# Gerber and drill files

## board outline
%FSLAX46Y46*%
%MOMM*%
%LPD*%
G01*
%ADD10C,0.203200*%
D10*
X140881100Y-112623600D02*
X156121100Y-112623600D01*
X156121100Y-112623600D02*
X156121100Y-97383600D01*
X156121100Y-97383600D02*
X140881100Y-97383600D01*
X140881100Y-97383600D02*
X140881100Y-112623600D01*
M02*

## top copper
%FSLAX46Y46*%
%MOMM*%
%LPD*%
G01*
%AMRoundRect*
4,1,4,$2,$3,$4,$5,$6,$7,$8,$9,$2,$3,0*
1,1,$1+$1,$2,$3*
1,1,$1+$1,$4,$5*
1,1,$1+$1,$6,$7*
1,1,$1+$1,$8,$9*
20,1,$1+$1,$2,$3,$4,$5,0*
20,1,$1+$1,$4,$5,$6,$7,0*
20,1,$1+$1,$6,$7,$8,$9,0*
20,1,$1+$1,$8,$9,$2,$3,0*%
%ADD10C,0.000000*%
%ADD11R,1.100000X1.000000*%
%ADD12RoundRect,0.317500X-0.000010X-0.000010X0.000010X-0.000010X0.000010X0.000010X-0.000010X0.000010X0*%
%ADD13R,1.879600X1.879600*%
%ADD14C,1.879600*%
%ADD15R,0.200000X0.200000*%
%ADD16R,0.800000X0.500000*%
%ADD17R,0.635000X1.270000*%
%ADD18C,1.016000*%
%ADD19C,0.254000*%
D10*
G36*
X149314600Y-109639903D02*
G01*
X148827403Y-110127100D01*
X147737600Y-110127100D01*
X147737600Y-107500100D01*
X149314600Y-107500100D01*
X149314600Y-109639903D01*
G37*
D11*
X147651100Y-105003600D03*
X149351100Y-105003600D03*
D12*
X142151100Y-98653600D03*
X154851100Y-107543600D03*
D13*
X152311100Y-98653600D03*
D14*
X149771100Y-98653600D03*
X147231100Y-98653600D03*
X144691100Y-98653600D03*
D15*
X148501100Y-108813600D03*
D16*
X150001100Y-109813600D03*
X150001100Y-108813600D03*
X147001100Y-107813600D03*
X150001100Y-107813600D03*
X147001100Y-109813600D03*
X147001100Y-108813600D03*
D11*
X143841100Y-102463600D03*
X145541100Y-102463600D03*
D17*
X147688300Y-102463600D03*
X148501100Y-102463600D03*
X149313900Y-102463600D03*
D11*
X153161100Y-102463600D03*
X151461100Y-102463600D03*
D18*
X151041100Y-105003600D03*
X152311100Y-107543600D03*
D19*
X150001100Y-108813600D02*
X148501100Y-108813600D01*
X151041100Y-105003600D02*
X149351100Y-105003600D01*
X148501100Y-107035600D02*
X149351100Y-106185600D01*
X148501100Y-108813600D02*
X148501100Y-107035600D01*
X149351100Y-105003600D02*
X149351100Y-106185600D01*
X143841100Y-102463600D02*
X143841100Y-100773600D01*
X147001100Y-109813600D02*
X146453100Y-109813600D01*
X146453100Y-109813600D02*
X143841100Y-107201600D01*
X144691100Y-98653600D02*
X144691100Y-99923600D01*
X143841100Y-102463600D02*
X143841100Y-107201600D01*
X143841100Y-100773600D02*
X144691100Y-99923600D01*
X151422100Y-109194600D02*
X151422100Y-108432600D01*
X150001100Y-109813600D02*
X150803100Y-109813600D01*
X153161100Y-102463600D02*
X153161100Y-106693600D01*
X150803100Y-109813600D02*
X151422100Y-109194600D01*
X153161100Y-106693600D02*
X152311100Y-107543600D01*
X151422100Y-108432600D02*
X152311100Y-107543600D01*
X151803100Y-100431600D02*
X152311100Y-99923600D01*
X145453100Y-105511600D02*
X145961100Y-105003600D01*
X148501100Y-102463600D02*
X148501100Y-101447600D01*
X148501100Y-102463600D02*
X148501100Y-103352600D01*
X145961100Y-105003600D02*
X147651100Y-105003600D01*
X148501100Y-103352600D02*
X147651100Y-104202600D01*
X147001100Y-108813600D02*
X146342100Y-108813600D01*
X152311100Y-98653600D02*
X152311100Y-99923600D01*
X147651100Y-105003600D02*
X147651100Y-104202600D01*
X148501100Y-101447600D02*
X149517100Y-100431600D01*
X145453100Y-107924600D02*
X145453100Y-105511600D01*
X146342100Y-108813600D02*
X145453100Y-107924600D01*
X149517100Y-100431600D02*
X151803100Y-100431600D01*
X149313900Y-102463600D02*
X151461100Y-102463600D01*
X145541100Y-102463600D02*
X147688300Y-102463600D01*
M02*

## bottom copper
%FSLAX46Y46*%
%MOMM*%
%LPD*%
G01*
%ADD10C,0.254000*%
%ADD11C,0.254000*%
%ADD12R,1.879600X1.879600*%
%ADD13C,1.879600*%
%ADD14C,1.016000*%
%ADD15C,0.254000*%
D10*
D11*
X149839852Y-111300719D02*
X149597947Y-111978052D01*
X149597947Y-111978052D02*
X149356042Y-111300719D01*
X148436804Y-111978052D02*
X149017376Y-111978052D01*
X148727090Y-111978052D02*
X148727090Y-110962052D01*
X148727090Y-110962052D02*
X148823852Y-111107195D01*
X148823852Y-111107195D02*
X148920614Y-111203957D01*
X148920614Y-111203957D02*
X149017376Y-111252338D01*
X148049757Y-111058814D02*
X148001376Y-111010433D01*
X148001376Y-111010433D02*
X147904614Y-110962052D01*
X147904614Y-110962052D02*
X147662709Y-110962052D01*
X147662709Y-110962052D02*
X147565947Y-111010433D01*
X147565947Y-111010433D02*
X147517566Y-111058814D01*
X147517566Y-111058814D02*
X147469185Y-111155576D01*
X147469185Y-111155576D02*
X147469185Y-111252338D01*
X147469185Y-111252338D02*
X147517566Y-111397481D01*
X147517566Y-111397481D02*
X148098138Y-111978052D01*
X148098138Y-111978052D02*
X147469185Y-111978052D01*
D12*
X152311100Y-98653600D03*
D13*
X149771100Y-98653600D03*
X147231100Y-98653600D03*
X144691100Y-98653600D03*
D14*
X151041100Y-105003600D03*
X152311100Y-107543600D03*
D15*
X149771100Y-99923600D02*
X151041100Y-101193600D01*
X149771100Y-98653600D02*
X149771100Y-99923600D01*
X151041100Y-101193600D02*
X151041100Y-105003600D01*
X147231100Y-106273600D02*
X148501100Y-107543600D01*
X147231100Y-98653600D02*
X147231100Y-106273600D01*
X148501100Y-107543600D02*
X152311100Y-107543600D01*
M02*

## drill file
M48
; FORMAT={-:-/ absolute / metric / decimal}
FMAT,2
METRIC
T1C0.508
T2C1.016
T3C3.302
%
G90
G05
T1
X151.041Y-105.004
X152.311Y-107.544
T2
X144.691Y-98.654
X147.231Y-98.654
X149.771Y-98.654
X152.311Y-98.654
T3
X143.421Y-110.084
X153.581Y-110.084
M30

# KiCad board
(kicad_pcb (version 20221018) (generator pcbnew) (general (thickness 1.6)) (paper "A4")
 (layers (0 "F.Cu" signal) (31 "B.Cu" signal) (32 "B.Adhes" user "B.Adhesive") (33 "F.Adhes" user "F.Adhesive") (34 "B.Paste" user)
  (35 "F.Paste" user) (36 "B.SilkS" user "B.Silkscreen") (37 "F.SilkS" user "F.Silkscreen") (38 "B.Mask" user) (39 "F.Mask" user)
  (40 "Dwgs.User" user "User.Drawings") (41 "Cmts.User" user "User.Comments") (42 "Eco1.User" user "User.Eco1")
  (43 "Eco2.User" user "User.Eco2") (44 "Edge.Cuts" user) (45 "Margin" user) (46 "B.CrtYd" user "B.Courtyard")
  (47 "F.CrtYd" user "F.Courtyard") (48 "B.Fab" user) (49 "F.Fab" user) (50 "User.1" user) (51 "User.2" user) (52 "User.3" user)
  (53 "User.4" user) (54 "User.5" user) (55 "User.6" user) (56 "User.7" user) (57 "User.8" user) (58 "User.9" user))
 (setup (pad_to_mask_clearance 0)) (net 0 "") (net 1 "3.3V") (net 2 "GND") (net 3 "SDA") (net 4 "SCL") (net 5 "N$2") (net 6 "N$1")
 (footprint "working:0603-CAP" (layer "F.Cu") (at 148.5011 105.0036)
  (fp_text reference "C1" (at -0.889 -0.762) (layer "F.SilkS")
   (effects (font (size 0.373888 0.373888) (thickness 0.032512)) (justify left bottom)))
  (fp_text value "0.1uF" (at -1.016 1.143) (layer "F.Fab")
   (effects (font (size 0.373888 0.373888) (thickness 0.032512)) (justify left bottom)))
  (pad "1" smd rect (at -0.85 0) (size 1.1 1) (layers "F.Cu" "F.Paste" "F.Mask") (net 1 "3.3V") (solder_mask_margin 0.1016)
   (thermal_bridge_angle 45))
  (pad "2" smd rect (at 0.85 0) (size 1.1 1) (layers "F.Cu" "F.Paste" "F.Mask") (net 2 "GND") (solder_mask_margin 0.1016)
   (thermal_bridge_angle 45)))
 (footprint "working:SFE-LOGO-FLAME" (layer "F.Cu") (at 153.42235 106.2101)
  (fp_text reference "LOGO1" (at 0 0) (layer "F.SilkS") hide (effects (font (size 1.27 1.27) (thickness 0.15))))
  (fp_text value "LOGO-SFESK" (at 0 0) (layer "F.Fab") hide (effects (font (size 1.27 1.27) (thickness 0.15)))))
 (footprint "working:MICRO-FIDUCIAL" (layer "F.Cu") (at 142.1511 98.6536)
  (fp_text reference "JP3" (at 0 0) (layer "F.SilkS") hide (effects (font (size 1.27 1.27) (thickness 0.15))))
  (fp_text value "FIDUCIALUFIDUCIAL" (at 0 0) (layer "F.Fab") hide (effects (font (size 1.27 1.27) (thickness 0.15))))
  (pad "1" smd roundrect (at 0 0) (size 0.635 0.635) (layers "F.Cu" "F.Mask") (roundrect_rratio 0.5) (solder_mask_margin 0.1016)
   (thermal_bridge_angle 45)))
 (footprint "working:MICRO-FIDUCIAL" (layer "F.Cu") (at 154.8511 107.5436)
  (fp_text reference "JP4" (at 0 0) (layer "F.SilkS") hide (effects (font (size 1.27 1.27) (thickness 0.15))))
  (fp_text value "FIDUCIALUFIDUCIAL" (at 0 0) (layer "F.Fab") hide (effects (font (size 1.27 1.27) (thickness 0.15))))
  (pad "1" smd roundrect (at 0 0) (size 0.635 0.635) (layers "F.Cu" "F.Mask") (roundrect_rratio 0.5) (solder_mask_margin 0.1016)
   (thermal_bridge_angle 45)))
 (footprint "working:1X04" (layer "F.Cu") (at 152.3111 98.6536 180)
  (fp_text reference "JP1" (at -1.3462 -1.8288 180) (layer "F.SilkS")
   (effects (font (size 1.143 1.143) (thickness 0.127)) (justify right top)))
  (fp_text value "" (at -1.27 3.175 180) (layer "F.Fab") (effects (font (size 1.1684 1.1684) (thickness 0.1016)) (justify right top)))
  (pad "1" thru_hole rect (at 0 0 270) (size 1.8796 1.8796) (drill 1.016) (layers "*.Cu" "*.Mask") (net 1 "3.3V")
   (solder_mask_margin 0.1016) (thermal_bridge_angle 45))
  (pad "2" thru_hole circle (at 2.54 0 270) (size 1.8796 1.8796) (drill 1.016) (layers "*.Cu" "*.Mask") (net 2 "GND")
   (solder_mask_margin 0.1016))
  (pad "3" thru_hole circle (at 5.08 0 270) (size 1.8796 1.8796) (drill 1.016) (layers "*.Cu" "*.Mask") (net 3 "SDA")
   (solder_mask_margin 0.1016))
  (pad "4" thru_hole circle (at 7.62 0 270) (size 1.8796 1.8796) (drill 1.016) (layers "*.Cu" "*.Mask") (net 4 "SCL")
   (solder_mask_margin 0.1016)))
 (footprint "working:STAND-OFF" (layer "F.Cu") (at 153.5811 110.0836)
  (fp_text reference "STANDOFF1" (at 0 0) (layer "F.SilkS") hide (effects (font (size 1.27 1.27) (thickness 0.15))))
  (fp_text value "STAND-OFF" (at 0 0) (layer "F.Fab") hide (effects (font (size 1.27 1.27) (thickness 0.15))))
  (pad "" np_thru_hole circle (at 0 0) (size 3.302 3.302) (drill 3.302) (layers "*.Cu" "*.Mask")))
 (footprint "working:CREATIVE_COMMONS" (layer "F.Cu") (at 128.1811 121.5136)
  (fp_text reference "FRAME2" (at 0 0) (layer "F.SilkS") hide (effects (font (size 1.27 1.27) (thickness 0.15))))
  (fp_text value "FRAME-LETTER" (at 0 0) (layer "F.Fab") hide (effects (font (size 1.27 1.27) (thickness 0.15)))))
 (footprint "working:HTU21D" (layer "F.Cu") (at 148.5011 108.8136)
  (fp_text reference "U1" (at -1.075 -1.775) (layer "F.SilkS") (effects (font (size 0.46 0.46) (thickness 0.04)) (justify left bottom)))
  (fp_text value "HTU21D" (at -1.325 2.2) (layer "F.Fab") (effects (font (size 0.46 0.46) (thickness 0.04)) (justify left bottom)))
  (fp_poly
   (pts (xy 0.8135 0.826303) (xy 0.326303 1.3135) (xy -0.7635 1.3135) (xy -0.7635 -1.3135) (xy 0.8135 -1.3135))
   (stroke (width 0) (type default)) (fill solid) (layer "F.Cu"))
  (pad "7" smd rect (at 0 0) (size 0.2 0.2) (layers "F.Cu" "F.Paste" "F.Mask") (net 2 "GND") (solder_mask_margin 0.1016)
   (thermal_bridge_angle 45))
  (pad "DATA" smd rect (at 1.5 1 270) (size 0.5 0.8) (layers "F.Cu" "F.Paste" "F.Mask") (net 3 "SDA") (solder_mask_margin 0.1016)
   (thermal_bridge_angle 45))
  (pad "GND" smd rect (at 1.5 0 270) (size 0.5 0.8) (layers "F.Cu" "F.Paste" "F.Mask") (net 2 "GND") (solder_mask_margin 0.1016)
   (thermal_bridge_angle 45))
  (pad "NC@1" smd rect (at -1.5 -1 270) (size 0.5 0.8) (layers "F.Cu" "F.Paste" "F.Mask") (solder_mask_margin 0.1016)
   (thermal_bridge_angle 45))
  (pad "NC@6" smd rect (at 1.5 -1 270) (size 0.5 0.8) (layers "F.Cu" "F.Paste" "F.Mask") (solder_mask_margin 0.1016)
   (thermal_bridge_angle 45))
  (pad "SCK" smd rect (at -1.5 1 270) (size 0.5 0.8) (layers "F.Cu" "F.Paste" "F.Mask") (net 4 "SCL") (solder_mask_margin 0.1016)
   (thermal_bridge_angle 45))
  (pad "VDD" smd rect (at -1.5 0 270) (size 0.5 0.8) (layers "F.Cu" "F.Paste" "F.Mask") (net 1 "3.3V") (solder_mask_margin 0.1016)
   (thermal_bridge_angle 45)))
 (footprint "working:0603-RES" (layer "F.Cu") (at 144.6911 102.4636)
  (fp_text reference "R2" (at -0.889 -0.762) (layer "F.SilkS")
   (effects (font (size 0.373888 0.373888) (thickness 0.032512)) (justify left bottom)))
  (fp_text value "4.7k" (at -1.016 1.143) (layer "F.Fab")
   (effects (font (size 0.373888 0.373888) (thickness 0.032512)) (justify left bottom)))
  (pad "1" smd rect (at -0.85 0) (size 1.1 1) (layers "F.Cu" "F.Paste" "F.Mask") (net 4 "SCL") (solder_mask_margin 0.1016)
   (thermal_bridge_angle 45))
  (pad "2" smd rect (at 0.85 0) (size 1.1 1) (layers "F.Cu" "F.Paste" "F.Mask") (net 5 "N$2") (solder_mask_margin 0.1016)
   (thermal_bridge_angle 45)))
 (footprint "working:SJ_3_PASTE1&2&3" (layer "F.Cu") (at 148.5011 102.4636)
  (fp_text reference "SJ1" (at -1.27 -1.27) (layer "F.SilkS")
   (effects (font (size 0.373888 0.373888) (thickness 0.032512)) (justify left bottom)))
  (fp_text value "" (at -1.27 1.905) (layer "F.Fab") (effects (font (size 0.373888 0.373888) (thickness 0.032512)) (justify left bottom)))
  (pad "1" smd rect (at -0.8128 0) (size 0.635 1.27) (layers "F.Cu" "F.Mask") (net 5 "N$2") (solder_mask_margin 0.1016)
   (thermal_bridge_angle 45))
  (pad "2" smd rect (at 0 0) (size 0.635 1.27) (layers "F.Cu" "F.Mask") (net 1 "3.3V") (solder_mask_margin 0.1016) (thermal_bridge_angle 45))
  (pad "3" smd rect (at 0.8128 0) (size 0.635 1.27) (layers "F.Cu" "F.Mask") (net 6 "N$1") (solder_mask_margin 0.1016)
   (thermal_bridge_angle 45)))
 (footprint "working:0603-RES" (layer "F.Cu") (at 152.3111 102.4636 180)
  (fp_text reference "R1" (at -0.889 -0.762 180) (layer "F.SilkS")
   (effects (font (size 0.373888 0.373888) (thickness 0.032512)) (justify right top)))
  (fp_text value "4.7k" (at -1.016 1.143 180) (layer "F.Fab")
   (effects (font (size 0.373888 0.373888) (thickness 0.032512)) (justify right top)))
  (pad "1" smd rect (at -0.85 0 180) (size 1.1 1) (layers "F.Cu" "F.Paste" "F.Mask") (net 3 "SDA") (solder_mask_margin 0.1016)
   (thermal_bridge_angle 45))
  (pad "2" smd rect (at 0.85 0 180) (size 1.1 1) (layers "F.Cu" "F.Paste" "F.Mask") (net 6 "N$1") (solder_mask_margin 0.1016)
   (thermal_bridge_angle 45)))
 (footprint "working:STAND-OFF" (layer "F.Cu") (at 143.4211 110.0836)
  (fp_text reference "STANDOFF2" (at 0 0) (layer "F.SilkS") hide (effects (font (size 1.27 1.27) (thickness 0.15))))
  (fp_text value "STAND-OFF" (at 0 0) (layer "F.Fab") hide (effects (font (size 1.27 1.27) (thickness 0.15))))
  (pad "" np_thru_hole circle (at 0 0) (size 3.302 3.302) (drill 3.302) (layers "*.Cu" "*.Mask")))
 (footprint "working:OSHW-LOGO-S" (layer "F.Cu") (at 142.7861 105.0036)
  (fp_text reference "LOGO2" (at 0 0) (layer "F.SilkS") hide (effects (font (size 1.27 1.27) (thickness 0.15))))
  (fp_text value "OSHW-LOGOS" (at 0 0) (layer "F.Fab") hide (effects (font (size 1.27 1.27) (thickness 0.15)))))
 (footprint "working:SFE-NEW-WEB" (layer "B.Cu") (at 154.5336 108.4961 180)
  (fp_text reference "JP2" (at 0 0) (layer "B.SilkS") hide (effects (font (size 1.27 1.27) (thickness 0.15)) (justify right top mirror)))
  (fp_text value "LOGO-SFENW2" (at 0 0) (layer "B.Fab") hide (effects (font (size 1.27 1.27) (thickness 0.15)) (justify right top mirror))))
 (gr_line (start 140.8811 112.6236) (end 156.1211 112.6236) (stroke (width 0.2032) (type solid)) (layer "Edge.Cuts"))
 (gr_line (start 156.1211 112.6236) (end 156.1211 97.3836) (stroke (width 0.2032) (type solid)) (layer "Edge.Cuts"))
 (gr_line (start 156.1211 97.3836) (end 140.8811 97.3836) (stroke (width 0.2032) (type solid)) (layer "Edge.Cuts"))
 (gr_line (start 140.8811 97.3836) (end 140.8811 112.6236) (stroke (width 0.2032) (type solid)) (layer "Edge.Cuts"))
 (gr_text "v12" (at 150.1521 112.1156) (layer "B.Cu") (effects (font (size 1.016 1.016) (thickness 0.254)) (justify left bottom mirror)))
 (segment (start 150.0011 108.8136) (end 148.5011 108.8136) (width 0.254) (layer "F.Cu") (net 2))
 (segment (start 151.0411 105.0036) (end 149.3511 105.0036) (width 0.254) (layer "F.Cu") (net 2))
 (segment (start 148.5011 107.0356) (end 149.3511 106.1856) (width 0.254) (layer "F.Cu") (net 2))
 (segment (start 148.5011 108.8136) (end 148.5011 107.0356) (width 0.254) (layer "F.Cu") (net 2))
 (segment (start 149.3511 105.0036) (end 149.3511 106.1856) (width 0.254) (layer "F.Cu") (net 2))
 (via (at 151.0411 105.0036) (size 1.016) (drill 0.508) (layers "F.Cu" "B.Cu") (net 2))
 (segment (start 149.7711 99.9236) (end 151.0411 101.1936) (width 0.254) (layer "B.Cu") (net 2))
 (segment (start 149.7711 98.6536) (end 149.7711 99.9236) (width 0.254) (layer "B.Cu") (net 2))
 (segment (start 151.0411 101.1936) (end 151.0411 105.0036) (width 0.254) (layer "B.Cu") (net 2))
 (segment (start 143.8411 102.4636) (end 143.8411 100.7736) (width 0.254) (layer "F.Cu") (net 4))
 (segment (start 147.0011 109.8136) (end 146.4531 109.8136) (width 0.254) (layer "F.Cu") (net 4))
 (segment (start 146.4531 109.8136) (end 143.8411 107.2016) (width 0.254) (layer "F.Cu") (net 4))
 (segment (start 144.6911 98.6536) (end 144.6911 99.9236) (width 0.254) (layer "F.Cu") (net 4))
 (segment (start 143.8411 102.4636) (end 143.8411 107.2016) (width 0.254) (layer "F.Cu") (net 4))
 (segment (start 143.8411 100.7736) (end 144.6911 99.9236) (width 0.254) (layer "F.Cu") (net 4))
 (segment (start 151.4221 109.1946) (end 151.4221 108.4326) (width 0.254) (layer "F.Cu") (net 3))
 (segment (start 150.0011 109.8136) (end 150.8031 109.8136) (width 0.254) (layer "F.Cu") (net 3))
 (segment (start 153.1611 102.4636) (end 153.1611 106.6936) (width 0.254) (layer "F.Cu") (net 3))
 (segment (start 150.8031 109.8136) (end 151.4221 109.1946) (width 0.254) (layer "F.Cu") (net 3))
 (segment (start 153.1611 106.6936) (end 152.3111 107.5436) (width 0.254) (layer "F.Cu") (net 3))
 (segment (start 151.4221 108.4326) (end 152.3111 107.5436) (width 0.254) (layer "F.Cu") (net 3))
 (via (at 152.3111 107.5436) (size 1.016) (drill 0.508) (layers "F.Cu" "B.Cu") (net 3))
 (segment (start 147.2311 106.2736) (end 148.5011 107.5436) (width 0.254) (layer "B.Cu") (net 3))
 (segment (start 147.2311 98.6536) (end 147.2311 106.2736) (width 0.254) (layer "B.Cu") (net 3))
 (segment (start 148.5011 107.5436) (end 152.3111 107.5436) (width 0.254) (layer "B.Cu") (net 3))
 (segment (start 151.8031 100.4316) (end 152.3111 99.9236) (width 0.254) (layer "F.Cu") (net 1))
 (segment (start 145.4531 105.5116) (end 145.9611 105.0036) (width 0.254) (layer "F.Cu") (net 1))
 (segment (start 148.5011 102.4636) (end 148.5011 101.4476) (width 0.254) (layer "F.Cu") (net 1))
 (segment (start 148.5011 102.4636) (end 148.5011 103.3526) (width 0.254) (layer "F.Cu") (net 1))
 (segment (start 145.9611 105.0036) (end 147.6511 105.0036) (width 0.254) (layer "F.Cu") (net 1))
 (segment (start 148.5011 103.3526) (end 147.6511 104.2026) (width 0.254) (layer "F.Cu") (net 1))
 (segment (start 147.0011 108.8136) (end 146.3421 108.8136) (width 0.254) (layer "F.Cu") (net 1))
 (segment (start 152.3111 98.6536) (end 152.3111 99.9236) (width 0.254) (layer "F.Cu") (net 1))
 (segment (start 147.6511 105.0036) (end 147.6511 104.2026) (width 0.254) (layer "F.Cu") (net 1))
 (segment (start 148.5011 101.4476) (end 149.5171 100.4316) (width 0.254) (layer "F.Cu") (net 1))
 (segment (start 145.4531 107.9246) (end 145.4531 105.5116) (width 0.254) (layer "F.Cu") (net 1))
 (segment (start 146.3421 108.8136) (end 145.4531 107.9246) (width 0.254) (layer "F.Cu") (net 1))
 (segment (start 149.5171 100.4316) (end 151.8031 100.4316) (width 0.254) (layer "F.Cu") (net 1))
 (segment (start 149.3139 102.4636) (end 151.4611 102.4636) (width 0.254) (layer "F.Cu") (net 6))
 (segment (start 145.5411 102.4636) (end 147.6883 102.4636) (width 0.254) (layer "F.Cu") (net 5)))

